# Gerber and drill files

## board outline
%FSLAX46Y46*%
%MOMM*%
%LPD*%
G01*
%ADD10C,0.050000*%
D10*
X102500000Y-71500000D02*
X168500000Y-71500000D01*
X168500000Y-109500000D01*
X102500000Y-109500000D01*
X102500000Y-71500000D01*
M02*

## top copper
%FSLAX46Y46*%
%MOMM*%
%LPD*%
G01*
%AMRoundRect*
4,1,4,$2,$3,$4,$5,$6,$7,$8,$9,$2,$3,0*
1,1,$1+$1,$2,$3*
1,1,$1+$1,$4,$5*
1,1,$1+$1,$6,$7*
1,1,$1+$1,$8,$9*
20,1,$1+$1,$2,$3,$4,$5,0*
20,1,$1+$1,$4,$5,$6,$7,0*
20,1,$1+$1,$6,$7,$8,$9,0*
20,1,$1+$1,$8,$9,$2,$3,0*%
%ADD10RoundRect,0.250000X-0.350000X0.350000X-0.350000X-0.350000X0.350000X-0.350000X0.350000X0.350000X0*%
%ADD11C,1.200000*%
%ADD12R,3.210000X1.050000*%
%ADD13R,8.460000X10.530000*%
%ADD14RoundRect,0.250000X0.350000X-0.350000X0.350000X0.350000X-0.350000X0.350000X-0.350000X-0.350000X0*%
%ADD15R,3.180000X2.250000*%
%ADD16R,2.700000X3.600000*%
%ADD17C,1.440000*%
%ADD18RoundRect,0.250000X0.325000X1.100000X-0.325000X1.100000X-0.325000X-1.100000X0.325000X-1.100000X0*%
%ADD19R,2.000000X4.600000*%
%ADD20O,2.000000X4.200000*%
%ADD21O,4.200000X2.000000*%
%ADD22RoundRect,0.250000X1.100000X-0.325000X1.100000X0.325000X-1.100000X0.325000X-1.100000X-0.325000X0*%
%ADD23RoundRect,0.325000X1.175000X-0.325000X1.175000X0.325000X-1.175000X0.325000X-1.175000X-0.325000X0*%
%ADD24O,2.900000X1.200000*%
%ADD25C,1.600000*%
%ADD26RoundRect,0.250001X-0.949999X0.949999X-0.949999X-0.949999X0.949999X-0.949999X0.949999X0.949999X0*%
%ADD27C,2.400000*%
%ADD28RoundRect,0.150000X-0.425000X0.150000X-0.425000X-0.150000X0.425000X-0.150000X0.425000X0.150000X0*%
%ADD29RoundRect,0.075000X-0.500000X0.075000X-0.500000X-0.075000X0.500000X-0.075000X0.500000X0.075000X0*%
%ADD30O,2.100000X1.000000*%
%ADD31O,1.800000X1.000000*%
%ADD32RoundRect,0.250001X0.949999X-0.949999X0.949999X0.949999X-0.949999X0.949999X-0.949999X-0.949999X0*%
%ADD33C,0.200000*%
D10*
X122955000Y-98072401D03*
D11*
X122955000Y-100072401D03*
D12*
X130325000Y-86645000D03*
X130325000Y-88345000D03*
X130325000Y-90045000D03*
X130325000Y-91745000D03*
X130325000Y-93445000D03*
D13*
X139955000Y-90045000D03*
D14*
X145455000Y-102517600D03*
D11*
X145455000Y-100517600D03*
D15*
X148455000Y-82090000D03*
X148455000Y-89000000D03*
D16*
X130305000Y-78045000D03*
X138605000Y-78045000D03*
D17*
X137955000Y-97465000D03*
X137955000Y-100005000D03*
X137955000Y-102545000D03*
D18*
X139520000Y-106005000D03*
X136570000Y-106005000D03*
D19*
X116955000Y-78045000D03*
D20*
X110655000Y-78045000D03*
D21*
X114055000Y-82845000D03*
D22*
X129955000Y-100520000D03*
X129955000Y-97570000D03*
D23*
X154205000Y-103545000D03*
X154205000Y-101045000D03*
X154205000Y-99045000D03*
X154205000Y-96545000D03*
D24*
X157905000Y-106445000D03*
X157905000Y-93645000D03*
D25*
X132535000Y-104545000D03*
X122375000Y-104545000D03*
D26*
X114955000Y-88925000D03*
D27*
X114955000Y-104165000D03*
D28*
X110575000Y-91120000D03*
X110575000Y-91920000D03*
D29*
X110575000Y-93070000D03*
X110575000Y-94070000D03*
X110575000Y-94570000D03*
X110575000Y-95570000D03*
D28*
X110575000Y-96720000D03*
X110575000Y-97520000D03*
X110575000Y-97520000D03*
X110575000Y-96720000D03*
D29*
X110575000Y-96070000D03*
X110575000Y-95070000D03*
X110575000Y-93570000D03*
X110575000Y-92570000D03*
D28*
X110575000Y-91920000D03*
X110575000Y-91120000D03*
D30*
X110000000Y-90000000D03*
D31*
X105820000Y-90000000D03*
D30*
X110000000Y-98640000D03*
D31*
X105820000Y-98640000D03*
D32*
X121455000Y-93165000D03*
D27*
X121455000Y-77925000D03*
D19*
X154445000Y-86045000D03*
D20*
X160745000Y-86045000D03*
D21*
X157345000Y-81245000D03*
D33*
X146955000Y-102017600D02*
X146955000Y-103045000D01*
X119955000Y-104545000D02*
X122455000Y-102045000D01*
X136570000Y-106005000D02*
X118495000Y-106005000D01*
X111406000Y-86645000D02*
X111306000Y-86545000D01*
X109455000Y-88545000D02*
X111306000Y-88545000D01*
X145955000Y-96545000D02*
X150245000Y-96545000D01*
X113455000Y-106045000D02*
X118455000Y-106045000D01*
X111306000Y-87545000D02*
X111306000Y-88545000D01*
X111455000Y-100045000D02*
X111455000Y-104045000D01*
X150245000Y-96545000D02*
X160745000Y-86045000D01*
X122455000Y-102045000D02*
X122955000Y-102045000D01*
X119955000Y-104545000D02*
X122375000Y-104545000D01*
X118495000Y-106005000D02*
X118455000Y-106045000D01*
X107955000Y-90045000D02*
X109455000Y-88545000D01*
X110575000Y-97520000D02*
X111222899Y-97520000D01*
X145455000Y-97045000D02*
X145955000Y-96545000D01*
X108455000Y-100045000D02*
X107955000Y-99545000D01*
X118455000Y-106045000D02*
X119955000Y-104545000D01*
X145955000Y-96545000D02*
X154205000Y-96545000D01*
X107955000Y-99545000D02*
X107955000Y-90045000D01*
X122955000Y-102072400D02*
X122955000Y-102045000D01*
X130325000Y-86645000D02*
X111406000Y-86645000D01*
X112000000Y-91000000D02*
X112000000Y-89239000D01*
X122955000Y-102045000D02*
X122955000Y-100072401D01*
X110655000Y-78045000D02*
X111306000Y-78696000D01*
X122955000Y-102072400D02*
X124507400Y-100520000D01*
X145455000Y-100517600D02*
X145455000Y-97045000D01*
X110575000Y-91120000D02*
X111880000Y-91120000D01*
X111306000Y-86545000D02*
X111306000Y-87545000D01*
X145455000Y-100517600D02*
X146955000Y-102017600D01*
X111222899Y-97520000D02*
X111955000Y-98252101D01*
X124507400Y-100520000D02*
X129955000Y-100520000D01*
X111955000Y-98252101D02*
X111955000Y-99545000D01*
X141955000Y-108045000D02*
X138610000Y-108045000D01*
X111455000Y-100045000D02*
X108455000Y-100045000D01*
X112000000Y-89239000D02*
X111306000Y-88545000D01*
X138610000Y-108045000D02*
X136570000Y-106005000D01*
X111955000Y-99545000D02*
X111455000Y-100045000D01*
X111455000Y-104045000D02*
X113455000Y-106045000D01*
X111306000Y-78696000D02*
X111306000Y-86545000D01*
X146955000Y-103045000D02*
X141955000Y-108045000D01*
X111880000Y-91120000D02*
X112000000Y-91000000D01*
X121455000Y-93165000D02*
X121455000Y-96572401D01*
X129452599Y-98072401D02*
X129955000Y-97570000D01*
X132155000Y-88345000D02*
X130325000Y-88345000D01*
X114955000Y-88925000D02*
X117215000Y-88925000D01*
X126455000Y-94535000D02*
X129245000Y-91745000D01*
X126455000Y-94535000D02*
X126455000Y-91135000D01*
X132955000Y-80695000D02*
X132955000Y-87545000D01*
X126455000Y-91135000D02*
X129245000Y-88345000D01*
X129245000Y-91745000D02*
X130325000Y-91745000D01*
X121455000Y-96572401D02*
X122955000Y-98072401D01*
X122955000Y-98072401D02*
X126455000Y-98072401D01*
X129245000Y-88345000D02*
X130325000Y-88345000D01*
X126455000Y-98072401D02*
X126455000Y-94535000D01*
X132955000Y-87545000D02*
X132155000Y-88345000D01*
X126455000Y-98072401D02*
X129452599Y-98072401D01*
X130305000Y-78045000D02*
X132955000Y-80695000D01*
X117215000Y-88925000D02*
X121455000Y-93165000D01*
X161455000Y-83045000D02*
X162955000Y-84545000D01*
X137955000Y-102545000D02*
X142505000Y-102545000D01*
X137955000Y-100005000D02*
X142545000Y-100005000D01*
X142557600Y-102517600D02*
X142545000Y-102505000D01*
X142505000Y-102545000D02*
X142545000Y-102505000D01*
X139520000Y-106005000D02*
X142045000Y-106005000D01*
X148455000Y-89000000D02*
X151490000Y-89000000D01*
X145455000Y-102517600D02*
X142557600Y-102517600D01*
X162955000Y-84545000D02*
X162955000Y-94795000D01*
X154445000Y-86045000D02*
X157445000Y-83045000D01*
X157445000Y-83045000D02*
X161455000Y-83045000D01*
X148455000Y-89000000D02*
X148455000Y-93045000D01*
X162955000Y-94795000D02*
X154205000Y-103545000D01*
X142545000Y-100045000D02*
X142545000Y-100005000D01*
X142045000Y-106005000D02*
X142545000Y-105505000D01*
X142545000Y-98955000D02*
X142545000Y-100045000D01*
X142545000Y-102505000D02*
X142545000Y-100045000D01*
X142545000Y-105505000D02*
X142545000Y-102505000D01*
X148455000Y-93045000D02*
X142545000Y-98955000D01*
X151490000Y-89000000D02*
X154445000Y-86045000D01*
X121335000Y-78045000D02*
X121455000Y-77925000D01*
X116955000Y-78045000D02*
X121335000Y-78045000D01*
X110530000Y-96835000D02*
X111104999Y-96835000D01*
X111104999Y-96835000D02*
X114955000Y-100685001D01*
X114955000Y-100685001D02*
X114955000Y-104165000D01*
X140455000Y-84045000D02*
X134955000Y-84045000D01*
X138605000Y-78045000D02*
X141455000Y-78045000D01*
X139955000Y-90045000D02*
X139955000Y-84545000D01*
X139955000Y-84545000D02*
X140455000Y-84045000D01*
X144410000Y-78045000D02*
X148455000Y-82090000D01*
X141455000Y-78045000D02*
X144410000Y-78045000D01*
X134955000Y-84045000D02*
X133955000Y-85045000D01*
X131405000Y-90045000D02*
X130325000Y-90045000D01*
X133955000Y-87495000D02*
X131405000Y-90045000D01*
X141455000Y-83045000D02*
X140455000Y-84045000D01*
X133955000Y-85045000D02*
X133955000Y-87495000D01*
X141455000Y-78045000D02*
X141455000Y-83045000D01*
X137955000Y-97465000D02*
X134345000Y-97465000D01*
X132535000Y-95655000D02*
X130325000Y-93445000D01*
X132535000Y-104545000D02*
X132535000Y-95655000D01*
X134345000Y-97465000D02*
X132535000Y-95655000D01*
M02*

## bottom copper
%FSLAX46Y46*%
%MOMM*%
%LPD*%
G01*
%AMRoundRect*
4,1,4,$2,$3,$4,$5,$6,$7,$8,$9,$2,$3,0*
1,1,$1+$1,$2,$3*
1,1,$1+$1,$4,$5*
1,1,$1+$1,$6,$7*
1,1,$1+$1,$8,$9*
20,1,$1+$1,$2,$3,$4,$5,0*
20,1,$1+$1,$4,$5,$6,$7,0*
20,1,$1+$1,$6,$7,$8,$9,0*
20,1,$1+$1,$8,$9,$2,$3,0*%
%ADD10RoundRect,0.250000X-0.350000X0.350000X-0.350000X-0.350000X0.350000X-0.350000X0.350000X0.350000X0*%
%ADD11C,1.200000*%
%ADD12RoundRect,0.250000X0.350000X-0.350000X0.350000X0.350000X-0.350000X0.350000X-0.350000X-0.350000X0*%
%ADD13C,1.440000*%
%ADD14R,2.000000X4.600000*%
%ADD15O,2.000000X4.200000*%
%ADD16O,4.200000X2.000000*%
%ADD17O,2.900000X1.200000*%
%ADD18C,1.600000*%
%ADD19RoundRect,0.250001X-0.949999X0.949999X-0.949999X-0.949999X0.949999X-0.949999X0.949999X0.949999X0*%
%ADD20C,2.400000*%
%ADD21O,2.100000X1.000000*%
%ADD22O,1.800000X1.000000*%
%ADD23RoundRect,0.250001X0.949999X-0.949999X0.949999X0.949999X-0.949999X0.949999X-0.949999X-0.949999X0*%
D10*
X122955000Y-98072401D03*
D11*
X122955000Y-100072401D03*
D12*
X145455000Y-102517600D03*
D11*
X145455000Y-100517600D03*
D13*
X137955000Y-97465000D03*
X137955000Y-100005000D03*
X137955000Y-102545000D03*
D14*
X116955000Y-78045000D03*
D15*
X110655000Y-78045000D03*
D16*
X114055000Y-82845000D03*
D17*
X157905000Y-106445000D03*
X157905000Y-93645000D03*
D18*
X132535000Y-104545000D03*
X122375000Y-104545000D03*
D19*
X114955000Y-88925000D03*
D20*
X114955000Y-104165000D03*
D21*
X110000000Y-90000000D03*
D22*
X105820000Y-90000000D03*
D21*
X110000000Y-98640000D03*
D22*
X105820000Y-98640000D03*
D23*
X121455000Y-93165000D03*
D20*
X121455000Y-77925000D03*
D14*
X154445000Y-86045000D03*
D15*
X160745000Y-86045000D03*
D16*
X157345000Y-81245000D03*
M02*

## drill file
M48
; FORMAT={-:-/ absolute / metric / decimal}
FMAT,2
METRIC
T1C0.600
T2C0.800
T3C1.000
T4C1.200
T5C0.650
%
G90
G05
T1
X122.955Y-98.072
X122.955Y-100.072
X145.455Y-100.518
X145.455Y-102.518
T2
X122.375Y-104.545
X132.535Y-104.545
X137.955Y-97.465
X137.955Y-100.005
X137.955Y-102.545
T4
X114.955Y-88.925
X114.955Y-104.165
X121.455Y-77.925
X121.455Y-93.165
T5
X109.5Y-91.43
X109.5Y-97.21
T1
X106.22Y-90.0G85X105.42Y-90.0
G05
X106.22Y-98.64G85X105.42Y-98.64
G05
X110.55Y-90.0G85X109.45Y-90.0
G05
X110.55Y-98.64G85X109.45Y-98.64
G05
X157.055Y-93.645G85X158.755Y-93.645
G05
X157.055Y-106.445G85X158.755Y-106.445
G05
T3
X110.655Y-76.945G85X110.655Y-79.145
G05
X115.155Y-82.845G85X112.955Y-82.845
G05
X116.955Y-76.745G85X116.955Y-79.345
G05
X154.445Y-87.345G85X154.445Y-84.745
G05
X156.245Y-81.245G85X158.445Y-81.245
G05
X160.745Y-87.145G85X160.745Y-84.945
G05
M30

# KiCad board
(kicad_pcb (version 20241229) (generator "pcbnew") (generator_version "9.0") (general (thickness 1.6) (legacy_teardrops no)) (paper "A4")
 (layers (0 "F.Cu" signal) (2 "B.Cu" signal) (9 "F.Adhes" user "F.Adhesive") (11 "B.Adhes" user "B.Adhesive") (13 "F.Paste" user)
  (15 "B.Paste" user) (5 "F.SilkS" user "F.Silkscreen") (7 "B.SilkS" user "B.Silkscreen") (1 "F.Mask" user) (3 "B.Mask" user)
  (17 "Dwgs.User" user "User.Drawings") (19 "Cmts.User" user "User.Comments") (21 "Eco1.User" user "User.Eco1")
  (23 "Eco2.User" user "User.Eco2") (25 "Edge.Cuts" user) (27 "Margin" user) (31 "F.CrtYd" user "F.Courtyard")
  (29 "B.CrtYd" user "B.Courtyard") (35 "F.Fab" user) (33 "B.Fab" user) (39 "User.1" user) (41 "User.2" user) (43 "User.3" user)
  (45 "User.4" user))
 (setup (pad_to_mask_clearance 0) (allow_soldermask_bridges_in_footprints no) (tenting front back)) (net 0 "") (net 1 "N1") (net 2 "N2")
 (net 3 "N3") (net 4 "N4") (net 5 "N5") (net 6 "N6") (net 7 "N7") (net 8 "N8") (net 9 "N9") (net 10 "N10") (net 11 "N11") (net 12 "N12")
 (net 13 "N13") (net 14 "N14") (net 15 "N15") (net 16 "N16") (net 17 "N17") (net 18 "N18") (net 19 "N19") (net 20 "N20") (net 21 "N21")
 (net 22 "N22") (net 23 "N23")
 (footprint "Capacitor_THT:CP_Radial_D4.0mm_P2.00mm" (layer "F.Cu") (at 122.955 98.072401 -90)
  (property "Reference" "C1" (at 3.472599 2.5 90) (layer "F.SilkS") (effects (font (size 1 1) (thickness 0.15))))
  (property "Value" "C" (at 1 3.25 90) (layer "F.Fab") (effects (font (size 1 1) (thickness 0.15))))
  (pad "1" thru_hole roundrect (at 0 0 270) (size 1.2 1.2) (drill 0.6) (layers "*.Cu" "*.Mask") (remove_unused_layers no)
   (roundrect_rratio 0.208333) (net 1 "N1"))
  (pad "2" thru_hole circle (at 2 0 270) (size 1.2 1.2) (drill 0.6) (layers "*.Cu" "*.Mask") (remove_unused_layers no) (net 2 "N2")))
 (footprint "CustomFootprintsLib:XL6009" (layer "F.Cu") (at 136.455 90.045)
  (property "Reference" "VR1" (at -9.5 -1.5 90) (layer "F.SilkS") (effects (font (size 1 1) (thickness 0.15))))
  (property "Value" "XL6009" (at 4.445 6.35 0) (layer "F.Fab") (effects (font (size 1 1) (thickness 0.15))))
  (pad "1" smd rect (at -6.13 -3.4) (size 3.21 1.05) (layers "F.Cu" "F.Mask" "F.Paste") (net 2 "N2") (solder_mask_margin 0.102))
  (pad "2" smd rect (at -6.13 -1.7) (size 3.21 1.05) (layers "F.Cu" "F.Mask" "F.Paste") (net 1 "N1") (solder_mask_margin 0.102))
  (pad "3" smd rect (at -6.13 0) (size 3.21 1.05) (layers "F.Cu" "F.Mask" "F.Paste") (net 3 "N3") (solder_mask_margin 0.102))
  (pad "4" smd rect (at -6.13 1.7) (size 3.21 1.05) (layers "F.Cu" "F.Mask" "F.Paste") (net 1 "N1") (solder_mask_margin 0.102))
  (pad "5" smd rect (at -6.13 3.4) (size 3.21 1.05) (layers "F.Cu" "F.Mask" "F.Paste") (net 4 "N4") (solder_mask_margin 0.102))
  (pad "6" smd rect (at 3.5 0) (size 8.46 10.53) (layers "F.Cu" "F.Mask") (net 3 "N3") (solder_mask_margin 0.102)))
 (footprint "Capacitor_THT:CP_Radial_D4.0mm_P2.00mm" (layer "F.Cu") (at 145.455 102.5176 90)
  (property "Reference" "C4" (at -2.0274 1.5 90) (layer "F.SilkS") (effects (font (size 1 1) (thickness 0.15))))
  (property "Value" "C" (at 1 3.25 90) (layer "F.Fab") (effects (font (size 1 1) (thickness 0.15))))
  (pad "1" thru_hole roundrect (at 0 0 90) (size 1.2 1.2) (drill 0.6) (layers "*.Cu" "*.Mask") (remove_unused_layers no)
   (roundrect_rratio 0.208333) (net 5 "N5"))
  (pad "2" thru_hole circle (at 2 0 90) (size 1.2 1.2) (drill 0.6) (layers "*.Cu" "*.Mask") (remove_unused_layers no) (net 2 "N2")))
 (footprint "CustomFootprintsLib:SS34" (layer "F.Cu") (at 148.455 85.545 90)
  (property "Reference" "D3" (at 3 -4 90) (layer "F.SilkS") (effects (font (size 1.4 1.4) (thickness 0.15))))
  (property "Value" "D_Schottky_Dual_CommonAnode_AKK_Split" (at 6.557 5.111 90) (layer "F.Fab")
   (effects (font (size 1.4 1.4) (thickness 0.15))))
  (pad "1" smd rect (at 3.455 0 90) (size 2.25 3.18) (layers "F.Cu" "F.Mask" "F.Paste") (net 3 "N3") (solder_mask_margin 0.102))
  (pad "2" smd rect (at -3.455 0 90) (size 2.25 3.18) (layers "F.Cu" "F.Mask" "F.Paste") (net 5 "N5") (solder_mask_margin 0.102)))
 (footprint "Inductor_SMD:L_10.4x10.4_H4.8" (layer "F.Cu") (at 134.455 78.045)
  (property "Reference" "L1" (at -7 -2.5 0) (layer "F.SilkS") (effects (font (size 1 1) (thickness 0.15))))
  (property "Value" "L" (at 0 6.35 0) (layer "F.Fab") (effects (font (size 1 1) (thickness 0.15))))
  (pad "1" smd rect (at -4.15 0) (size 2.7 3.6) (layers "F.Cu" "F.Mask" "F.Paste") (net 1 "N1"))
  (pad "2" smd rect (at 4.15 0) (size 2.7 3.6) (layers "F.Cu" "F.Mask" "F.Paste") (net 3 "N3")))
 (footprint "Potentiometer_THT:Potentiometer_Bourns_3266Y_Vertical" (layer "F.Cu") (at 137.955 97.465 90)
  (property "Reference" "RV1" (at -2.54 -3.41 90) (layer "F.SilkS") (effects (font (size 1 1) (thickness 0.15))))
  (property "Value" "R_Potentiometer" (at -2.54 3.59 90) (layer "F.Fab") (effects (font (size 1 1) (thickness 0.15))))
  (pad "1" thru_hole circle (at 0 0 90) (size 1.44 1.44) (drill 0.8) (layers "*.Cu" "*.Mask") (remove_unused_layers no) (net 4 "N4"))
  (pad "2" thru_hole circle (at -2.54 0 90) (size 1.44 1.44) (drill 0.8) (layers "*.Cu" "*.Mask") (remove_unused_layers no) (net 5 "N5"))
  (pad "3" thru_hole circle (at -5.08 0 90) (size 1.44 1.44) (drill 0.8) (layers "*.Cu" "*.Mask") (remove_unused_layers no) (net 5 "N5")))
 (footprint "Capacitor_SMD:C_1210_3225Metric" (layer "F.Cu") (at 138.045 106.005 180)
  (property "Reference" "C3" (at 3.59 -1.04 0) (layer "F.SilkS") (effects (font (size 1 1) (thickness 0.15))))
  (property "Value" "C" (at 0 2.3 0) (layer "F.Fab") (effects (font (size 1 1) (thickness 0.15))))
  (pad "1" smd roundrect (at -1.475 0 180) (size 1.15 2.7) (layers "F.Cu" "F.Mask" "F.Paste") (roundrect_rratio 0.217391) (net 5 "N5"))
  (pad "2" smd roundrect (at 1.475 0 180) (size 1.15 2.7) (layers "F.Cu" "F.Mask" "F.Paste") (roundrect_rratio 0.217391) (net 2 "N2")))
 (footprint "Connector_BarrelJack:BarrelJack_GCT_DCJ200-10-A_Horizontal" (layer "F.Cu") (at 116.955 78.045 -90)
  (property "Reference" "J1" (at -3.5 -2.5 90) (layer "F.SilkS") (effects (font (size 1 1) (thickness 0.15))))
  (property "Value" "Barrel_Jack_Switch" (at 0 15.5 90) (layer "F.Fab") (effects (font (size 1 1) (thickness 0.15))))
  (pad "1" thru_hole rect (at 0 0 270) (size 4.6 2) (drill oval 3.6 1) (layers "*.Cu" "*.Mask") (remove_unused_layers no) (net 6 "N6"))
  (pad "2" thru_hole oval (at 0 6.3 270) (size 4.2 2) (drill oval 3.2 1) (layers "*.Cu" "*.Mask") (remove_unused_layers no) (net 2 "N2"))
  (pad "3" thru_hole oval (at 4.8 2.9 270) (size 2 4.2) (drill oval 1 3.2) (layers "*.Cu" "*.Mask") (remove_unused_layers no) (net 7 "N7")))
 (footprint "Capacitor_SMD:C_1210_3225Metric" (layer "F.Cu") (at 129.955 99.045 90)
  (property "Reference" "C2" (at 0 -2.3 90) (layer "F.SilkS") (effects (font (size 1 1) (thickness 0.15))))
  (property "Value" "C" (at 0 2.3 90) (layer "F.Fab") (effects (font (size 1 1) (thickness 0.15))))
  (pad "1" smd roundrect (at -1.475 0 90) (size 1.15 2.7) (layers "F.Cu" "F.Mask" "F.Paste") (roundrect_rratio 0.217391) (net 2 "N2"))
  (pad "2" smd roundrect (at 1.475 0 90) (size 1.15 2.7) (layers "F.Cu" "F.Mask" "F.Paste") (roundrect_rratio 0.217391) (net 1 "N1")))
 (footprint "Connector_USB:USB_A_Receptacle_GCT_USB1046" (layer "F.Cu") (at 161.455 100.045 90)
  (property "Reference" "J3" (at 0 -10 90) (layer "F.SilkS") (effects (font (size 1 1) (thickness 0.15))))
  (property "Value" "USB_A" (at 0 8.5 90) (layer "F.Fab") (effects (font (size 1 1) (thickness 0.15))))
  (pad "" smd oval (at -6.4 -3.55 90) (size 1.2 2.9) (layers "F.Paste") (thermal_bridge_angle 45))
  (pad "" smd oval (at 6.4 -3.55 90) (size 1.2 2.9) (layers "F.Paste") (thermal_bridge_angle 45))
  (pad "1" smd roundrect (at -3.5 -7.25 90) (size 1.3 3) (layers "F.Cu" "F.Mask" "F.Paste") (roundrect_rratio 0.25) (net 5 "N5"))
  (pad "2" smd roundrect (at -1 -7.25 90) (size 1.3 3) (layers "F.Cu" "F.Mask" "F.Paste") (roundrect_rratio 0.25) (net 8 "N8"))
  (pad "3" smd roundrect (at 1 -7.25 90) (size 1.3 3) (layers "F.Cu" "F.Mask" "F.Paste") (roundrect_rratio 0.25) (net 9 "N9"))
  (pad "4" smd roundrect (at 3.5 -7.25 90) (size 1.3 3) (layers "F.Cu" "F.Mask" "F.Paste") (roundrect_rratio 0.25) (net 2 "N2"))
  (pad "5" thru_hole oval (at -6.4 -3.55 90) (size 1.2 2.9) (drill oval 0.6 2.3) (layers "*.Cu" "*.Mask") (remove_unused_layers no)
   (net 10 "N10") (thermal_bridge_angle 45))
  (pad "5" thru_hole oval (at 6.4 -3.55 90) (size 1.2 2.9) (drill oval 0.6 2.3) (layers "*.Cu" "*.Mask") (remove_unused_layers no)
   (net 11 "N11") (thermal_bridge_angle 45)))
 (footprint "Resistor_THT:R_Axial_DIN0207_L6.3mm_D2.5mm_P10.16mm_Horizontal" (layer "F.Cu") (at 132.535 104.545 180)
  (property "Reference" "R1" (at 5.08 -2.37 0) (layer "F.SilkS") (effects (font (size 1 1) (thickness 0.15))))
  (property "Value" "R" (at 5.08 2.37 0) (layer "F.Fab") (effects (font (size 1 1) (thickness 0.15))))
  (pad "1" thru_hole circle (at 0 0 180) (size 1.6 1.6) (drill 0.8) (layers "*.Cu" "*.Mask") (remove_unused_layers no) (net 4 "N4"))
  (pad "2" thru_hole circle (at 10.16 0 180) (size 1.6 1.6) (drill 0.8) (layers "*.Cu" "*.Mask") (remove_unused_layers no) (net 2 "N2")))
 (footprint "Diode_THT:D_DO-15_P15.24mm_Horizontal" (layer "F.Cu") (at 114.955 88.925 -90)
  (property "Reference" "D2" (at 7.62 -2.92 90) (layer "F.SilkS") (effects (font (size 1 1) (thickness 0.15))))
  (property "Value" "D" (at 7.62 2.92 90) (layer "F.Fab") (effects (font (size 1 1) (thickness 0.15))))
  (pad "1" thru_hole roundrect (at 0 0 270) (size 2.4 2.4) (drill 1.2) (layers "*.Cu" "*.Mask") (remove_unused_layers no)
   (roundrect_rratio 0.104167) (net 1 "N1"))
  (pad "2" thru_hole circle (at 15.24 0 270) (size 2.4 2.4) (drill 1.2) (layers "*.Cu" "*.Mask") (remove_unused_layers no) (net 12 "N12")))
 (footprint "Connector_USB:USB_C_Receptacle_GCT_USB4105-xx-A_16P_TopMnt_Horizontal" (layer "F.Cu") (at 106.895 94.32 -90)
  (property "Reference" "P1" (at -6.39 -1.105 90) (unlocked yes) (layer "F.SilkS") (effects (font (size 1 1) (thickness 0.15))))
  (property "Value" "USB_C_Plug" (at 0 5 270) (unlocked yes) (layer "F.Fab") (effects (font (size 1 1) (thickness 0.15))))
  (pad "" np_thru_hole circle (at -2.89 -2.605 270) (size 0.65 0.65) (drill 0.65) (layers "*.Cu" "*.Mask"))
  (pad "" np_thru_hole circle (at 2.89 -2.605 270) (size 0.65 0.65) (drill 0.65) (layers "*.Cu" "*.Mask"))
  (pad "A1" smd roundrect (at -3.2 -3.68 270) (size 0.6 1.15) (layers "F.Cu" "F.Mask" "F.Paste") (roundrect_rratio 0.25) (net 2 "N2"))
  (pad "A4" smd roundrect (at -2.4 -3.68 270) (size 0.6 1.15) (layers "F.Cu" "F.Mask" "F.Paste") (roundrect_rratio 0.25) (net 12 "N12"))
  (pad "A5" smd roundrect (at -1.25 -3.68 270) (size 0.3 1.15) (layers "F.Cu" "F.Mask" "F.Paste") (roundrect_rratio 0.25) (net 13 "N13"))
  (pad "A6" smd roundrect (at -0.25 -3.68 270) (size 0.3 1.15) (layers "F.Cu" "F.Mask" "F.Paste") (roundrect_rratio 0.25) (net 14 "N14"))
  (pad "A7" smd roundrect (at 0.25 -3.68 270) (size 0.3 1.15) (layers "F.Cu" "F.Mask" "F.Paste") (roundrect_rratio 0.25) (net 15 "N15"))
  (pad "A8" smd roundrect (at 1.25 -3.68 270) (size 0.3 1.15) (layers "F.Cu" "F.Mask" "F.Paste") (roundrect_rratio 0.25) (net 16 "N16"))
  (pad "A9" smd roundrect (at 2.4 -3.68 270) (size 0.6 1.15) (layers "F.Cu" "F.Mask" "F.Paste") (roundrect_rratio 0.25) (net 12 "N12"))
  (pad "A12" smd roundrect (at 3.2 -3.68 270) (size 0.6 1.15) (layers "F.Cu" "F.Mask" "F.Paste") (roundrect_rratio 0.25) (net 2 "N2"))
  (pad "B1" smd roundrect (at 3.2 -3.68 270) (size 0.6 1.15) (layers "F.Cu" "F.Mask" "F.Paste") (roundrect_rratio 0.25) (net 2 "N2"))
  (pad "B4" smd roundrect (at 2.4 -3.68 270) (size 0.6 1.15) (layers "F.Cu" "F.Mask" "F.Paste") (roundrect_rratio 0.25) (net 12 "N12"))
  (pad "B5" smd roundrect (at 1.75 -3.68 270) (size 0.3 1.15) (layers "F.Cu" "F.Mask" "F.Paste") (roundrect_rratio 0.25) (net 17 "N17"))
  (pad "B6" smd roundrect (at 0.75 -3.68 270) (size 0.3 1.15) (layers "F.Cu" "F.Mask" "F.Paste") (roundrect_rratio 0.25))
  (pad "B7" smd roundrect (at -0.75 -3.68 270) (size 0.3 1.15) (layers "F.Cu" "F.Mask" "F.Paste") (roundrect_rratio 0.25))
  (pad "B8" smd roundrect (at -1.75 -3.68 270) (size 0.3 1.15) (layers "F.Cu" "F.Mask" "F.Paste") (roundrect_rratio 0.25) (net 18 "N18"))
  (pad "B9" smd roundrect (at -2.4 -3.68 270) (size 0.6 1.15) (layers "F.Cu" "F.Mask" "F.Paste") (roundrect_rratio 0.25) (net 12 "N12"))
  (pad "B12" smd roundrect (at -3.2 -3.68 270) (size 0.6 1.15) (layers "F.Cu" "F.Mask" "F.Paste") (roundrect_rratio 0.25) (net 2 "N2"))
  (pad "S1" thru_hole oval (at -4.32 -3.105 270) (size 1 2.1) (drill oval 0.6 1.7) (layers "*.Cu" "*.Mask" "F.Paste")
   (remove_unused_layers no) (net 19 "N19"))
  (pad "S1" thru_hole oval (at -4.32 1.075 270) (size 1 1.8) (drill oval 0.6 1.4) (layers "*.Cu" "*.Mask" "F.Paste")
   (remove_unused_layers no) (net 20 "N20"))
  (pad "S1" thru_hole oval (at 4.32 -3.105 270) (size 1 2.1) (drill oval 0.6 1.7) (layers "*.Cu" "*.Mask" "F.Paste")
   (remove_unused_layers no) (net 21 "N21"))
  (pad "S1" thru_hole oval (at 4.32 1.075 270) (size 1 1.8) (drill oval 0.6 1.4) (layers "*.Cu" "*.Mask" "F.Paste")
   (remove_unused_layers no) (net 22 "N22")))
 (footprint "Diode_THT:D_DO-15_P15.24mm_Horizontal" (layer "F.Cu") (at 121.455 93.165 90)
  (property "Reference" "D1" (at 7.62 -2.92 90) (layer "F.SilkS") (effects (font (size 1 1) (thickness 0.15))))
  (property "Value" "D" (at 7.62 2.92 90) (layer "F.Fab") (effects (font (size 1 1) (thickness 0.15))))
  (pad "1" thru_hole roundrect (at 0 0 90) (size 2.4 2.4) (drill 1.2) (layers "*.Cu" "*.Mask") (remove_unused_layers no)
   (roundrect_rratio 0.104167) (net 1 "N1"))
  (pad "2" thru_hole circle (at 15.24 0 90) (size 2.4 2.4) (drill 1.2) (layers "*.Cu" "*.Mask") (remove_unused_layers no) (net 6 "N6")))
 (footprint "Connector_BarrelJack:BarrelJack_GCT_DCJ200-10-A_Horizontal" (layer "F.Cu") (at 154.445 86.045 90)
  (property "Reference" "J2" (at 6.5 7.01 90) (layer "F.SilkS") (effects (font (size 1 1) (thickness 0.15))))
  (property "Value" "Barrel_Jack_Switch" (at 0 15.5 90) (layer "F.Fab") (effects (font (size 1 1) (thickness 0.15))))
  (pad "1" thru_hole rect (at 0 0 90) (size 4.6 2) (drill oval 3.6 1) (layers "*.Cu" "*.Mask") (remove_unused_layers no) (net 5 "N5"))
  (pad "2" thru_hole oval (at 0 6.3 90) (size 4.2 2) (drill oval 3.2 1) (layers "*.Cu" "*.Mask") (remove_unused_layers no) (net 2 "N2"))
  (pad "3" thru_hole oval (at 4.8 2.9 90) (size 2 4.2) (drill oval 1 3.2) (layers "*.Cu" "*.Mask") (remove_unused_layers no) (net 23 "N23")))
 (gr_rect (start 102.5 71.5) (end 168.5 109.5) (stroke (width 0.05) (type default)) (fill no) (layer "Edge.Cuts"))
 (segment (start 146.955 102.0176) (end 146.955 103.045) (width 0.2) (layer "F.Cu") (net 2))
 (segment (start 119.955 104.545) (end 122.455 102.045) (width 0.2) (layer "F.Cu") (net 2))
 (segment (start 136.57 106.005) (end 118.495 106.005) (width 0.2) (layer "F.Cu") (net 2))
 (segment (start 111.406 86.645) (end 111.306 86.545) (width 0.2) (layer "F.Cu") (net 2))
 (segment (start 109.455 88.545) (end 111.306 88.545) (width 0.2) (layer "F.Cu") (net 2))
 (segment (start 145.955 96.545) (end 150.245 96.545) (width 0.2) (layer "F.Cu") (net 2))
 (segment (start 113.455 106.045) (end 118.455 106.045) (width 0.2) (layer "F.Cu") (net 2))
 (segment (start 111.306 87.545) (end 111.306 88.545) (width 0.2) (layer "F.Cu") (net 2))
 (segment (start 111.455 100.045) (end 111.455 104.045) (width 0.2) (layer "F.Cu") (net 2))
 (segment (start 150.245 96.545) (end 160.745 86.045) (width 0.2) (layer "F.Cu") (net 2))
 (segment (start 122.455 102.045) (end 122.955 102.045) (width 0.2) (layer "F.Cu") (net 2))
 (segment (start 119.955 104.545) (end 122.375 104.545) (width 0.2) (layer "F.Cu") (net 2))
 (segment (start 118.495 106.005) (end 118.455 106.045) (width 0.2) (layer "F.Cu") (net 2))
 (segment (start 107.955 90.045) (end 109.455 88.545) (width 0.2) (layer "F.Cu") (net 2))
 (segment (start 110.575 97.52) (end 111.222899 97.52) (width 0.2) (layer "F.Cu") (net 2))
 (segment (start 145.455 97.045) (end 145.955 96.545) (width 0.2) (layer "F.Cu") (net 2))
 (segment (start 108.455 100.045) (end 107.955 99.545) (width 0.2) (layer "F.Cu") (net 2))
 (segment (start 118.455 106.045) (end 119.955 104.545) (width 0.2) (layer "F.Cu") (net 2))
 (segment (start 145.955 96.545) (end 154.205 96.545) (width 0.2) (layer "F.Cu") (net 2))
 (segment (start 107.955 99.545) (end 107.955 90.045) (width 0.2) (layer "F.Cu") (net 2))
 (segment (start 122.955 102.0724) (end 122.955 102.045) (width 0.2) (layer "F.Cu") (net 2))
 (segment (start 130.325 86.645) (end 111.406 86.645) (width 0.2) (layer "F.Cu") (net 2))
 (segment (start 112 91) (end 112 89.239) (width 0.2) (layer "F.Cu") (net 2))
 (segment (start 122.955 102.045) (end 122.955 100.072401) (width 0.2) (layer "F.Cu") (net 2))
 (segment (start 110.655 78.045) (end 111.306 78.696) (width 0.2) (layer "F.Cu") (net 2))
 (segment (start 122.955 102.0724) (end 124.5074 100.52) (width 0.2) (layer "F.Cu") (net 2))
 (segment (start 145.455 100.5176) (end 145.455 97.045) (width 0.2) (layer "F.Cu") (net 2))
 (segment (start 110.575 91.12) (end 111.88 91.12) (width 0.2) (layer "F.Cu") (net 2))
 (segment (start 111.306 86.545) (end 111.306 87.545) (width 0.2) (layer "F.Cu") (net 2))
 (segment (start 145.455 100.5176) (end 146.955 102.0176) (width 0.2) (layer "F.Cu") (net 2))
 (segment (start 111.222899 97.52) (end 111.955 98.252101) (width 0.2) (layer "F.Cu") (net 2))
 (segment (start 124.5074 100.52) (end 129.955 100.52) (width 0.2) (layer "F.Cu") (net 2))
 (segment (start 111.955 98.252101) (end 111.955 99.545) (width 0.2) (layer "F.Cu") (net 2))
 (segment (start 141.955 108.045) (end 138.61 108.045) (width 0.2) (layer "F.Cu") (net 2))
 (segment (start 111.455 100.045) (end 108.455 100.045) (width 0.2) (layer "F.Cu") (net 2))
 (segment (start 112 89.239) (end 111.306 88.545) (width 0.2) (layer "F.Cu") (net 2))
 (segment (start 138.61 108.045) (end 136.57 106.005) (width 0.2) (layer "F.Cu") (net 2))
 (segment (start 111.955 99.545) (end 111.455 100.045) (width 0.2) (layer "F.Cu") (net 2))
 (segment (start 111.455 104.045) (end 113.455 106.045) (width 0.2) (layer "F.Cu") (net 2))
 (segment (start 111.306 78.696) (end 111.306 86.545) (width 0.2) (layer "F.Cu") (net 2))
 (segment (start 146.955 103.045) (end 141.955 108.045) (width 0.2) (layer "F.Cu") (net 2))
 (segment (start 111.88 91.12) (end 112 91) (width 0.2) (layer "F.Cu") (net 2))
 (segment (start 121.455 93.165) (end 121.455 96.572401) (width 0.2) (layer "F.Cu") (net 1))
 (segment (start 129.452599 98.072401) (end 129.955 97.57) (width 0.2) (layer "F.Cu") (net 1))
 (segment (start 132.155 88.345) (end 130.325 88.345) (width 0.2) (layer "F.Cu") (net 1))
 (segment (start 114.955 88.925) (end 117.215 88.925) (width 0.2) (layer "F.Cu") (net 1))
 (segment (start 126.455 94.535) (end 129.245 91.745) (width 0.2) (layer "F.Cu") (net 1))
 (segment (start 126.455 94.535) (end 126.455 91.135) (width 0.2) (layer "F.Cu") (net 1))
 (segment (start 132.955 80.695) (end 132.955 87.545) (width 0.2) (layer "F.Cu") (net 1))
 (segment (start 126.455 91.135) (end 129.245 88.345) (width 0.2) (layer "F.Cu") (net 1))
 (segment (start 129.245 91.745) (end 130.325 91.745) (width 0.2) (layer "F.Cu") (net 1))
 (segment (start 121.455 96.572401) (end 122.955 98.072401) (width 0.2) (layer "F.Cu") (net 1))
 (segment (start 122.955 98.072401) (end 126.455 98.072401) (width 0.2) (layer "F.Cu") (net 1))
 (segment (start 129.245 88.345) (end 130.325 88.345) (width 0.2) (layer "F.Cu") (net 1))
 (segment (start 126.455 98.072401) (end 126.455 94.535) (width 0.2) (layer "F.Cu") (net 1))
 (segment (start 132.955 87.545) (end 132.155 88.345) (width 0.2) (layer "F.Cu") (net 1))
 (segment (start 126.455 98.072401) (end 129.452599 98.072401) (width 0.2) (layer "F.Cu") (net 1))
 (segment (start 130.305 78.045) (end 132.955 80.695) (width 0.2) (layer "F.Cu") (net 1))
 (segment (start 117.215 88.925) (end 121.455 93.165) (width 0.2) (layer "F.Cu") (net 1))
 (segment (start 161.455 83.045) (end 162.955 84.545) (width 0.2) (layer "F.Cu") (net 5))
 (segment (start 137.955 102.545) (end 142.505 102.545) (width 0.2) (layer "F.Cu") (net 5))
 (segment (start 137.955 100.005) (end 142.545 100.005) (width 0.2) (layer "F.Cu") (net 5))
 (segment (start 142.5576 102.5176) (end 142.545 102.505) (width 0.2) (layer "F.Cu") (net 5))
 (segment (start 142.505 102.545) (end 142.545 102.505) (width 0.2) (layer "F.Cu") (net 5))
 (segment (start 139.52 106.005) (end 142.045 106.005) (width 0.2) (layer "F.Cu") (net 5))
 (segment (start 148.455 89) (end 151.49 89) (width 0.2) (layer "F.Cu") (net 5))
 (segment (start 145.455 102.5176) (end 142.5576 102.5176) (width 0.2) (layer "F.Cu") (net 5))
 (segment (start 162.955 84.545) (end 162.955 94.795) (width 0.2) (layer "F.Cu") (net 5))
 (segment (start 154.445 86.045) (end 157.445 83.045) (width 0.2) (layer "F.Cu") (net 5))
 (segment (start 157.445 83.045) (end 161.455 83.045) (width 0.2) (layer "F.Cu") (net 5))
 (segment (start 148.455 89) (end 148.455 93.045) (width 0.2) (layer "F.Cu") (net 5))
 (segment (start 162.955 94.795) (end 154.205 103.545) (width 0.2) (layer "F.Cu") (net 5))
 (segment (start 142.545 100.045) (end 142.545 100.005) (width 0.2) (layer "F.Cu") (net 5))
 (segment (start 142.045 106.005) (end 142.545 105.505) (width 0.2) (layer "F.Cu") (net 5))
 (segment (start 142.545 98.955) (end 142.545 100.045) (width 0.2) (layer "F.Cu") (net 5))
 (segment (start 142.545 102.505) (end 142.545 100.045) (width 0.2) (layer "F.Cu") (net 5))
 (segment (start 142.545 105.505) (end 142.545 102.505) (width 0.2) (layer "F.Cu") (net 5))
 (segment (start 148.455 93.045) (end 142.545 98.955) (width 0.2) (layer "F.Cu") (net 5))
 (segment (start 151.49 89) (end 154.445 86.045) (width 0.2) (layer "F.Cu") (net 5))
 (segment (start 121.335 78.045) (end 121.455 77.925) (width 0.2) (layer "F.Cu") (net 6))
 (segment (start 116.955 78.045) (end 121.335 78.045) (width 0.2) (layer "F.Cu") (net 6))
 (segment (start 110.53 96.835) (end 111.104999 96.835) (width 0.2) (layer "F.Cu") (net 12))
 (segment (start 111.104999 96.835) (end 114.955 100.685001) (width 0.2) (layer "F.Cu") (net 12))
 (segment (start 114.955 100.685001) (end 114.955 104.165) (width 0.2) (layer "F.Cu") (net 12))
 (segment (start 140.455 84.045) (end 134.955 84.045) (width 0.2) (layer "F.Cu") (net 3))
 (segment (start 138.605 78.045) (end 141.455 78.045) (width 0.2) (layer "F.Cu") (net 3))
 (segment (start 139.955 90.045) (end 139.955 84.545) (width 0.2) (layer "F.Cu") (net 3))
 (segment (start 139.955 84.545) (end 140.455 84.045) (width 0.2) (layer "F.Cu") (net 3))
 (segment (start 144.41 78.045) (end 148.455 82.09) (width 0.2) (layer "F.Cu") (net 3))
 (segment (start 141.455 78.045) (end 144.41 78.045) (width 0.2) (layer "F.Cu") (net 3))
 (segment (start 134.955 84.045) (end 133.955 85.045) (width 0.2) (layer "F.Cu") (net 3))
 (segment (start 131.405 90.045) (end 130.325 90.045) (width 0.2) (layer "F.Cu") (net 3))
 (segment (start 133.955 87.495) (end 131.405 90.045) (width 0.2) (layer "F.Cu") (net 3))
 (segment (start 141.455 83.045) (end 140.455 84.045) (width 0.2) (layer "F.Cu") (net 3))
 (segment (start 133.955 85.045) (end 133.955 87.495) (width 0.2) (layer "F.Cu") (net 3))
 (segment (start 141.455 78.045) (end 141.455 83.045) (width 0.2) (layer "F.Cu") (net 3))
 (segment (start 137.955 97.465) (end 134.345 97.465) (width 0.2) (layer "F.Cu") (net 4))
 (segment (start 132.535 95.655) (end 130.325 93.445) (width 0.2) (layer "F.Cu") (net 4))
 (segment (start 132.535 104.545) (end 132.535 95.655) (width 0.2) (layer "F.Cu") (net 4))
 (segment (start 134.345 97.465) (end 132.535 95.655) (width 0.2) (layer "F.Cu") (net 4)))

